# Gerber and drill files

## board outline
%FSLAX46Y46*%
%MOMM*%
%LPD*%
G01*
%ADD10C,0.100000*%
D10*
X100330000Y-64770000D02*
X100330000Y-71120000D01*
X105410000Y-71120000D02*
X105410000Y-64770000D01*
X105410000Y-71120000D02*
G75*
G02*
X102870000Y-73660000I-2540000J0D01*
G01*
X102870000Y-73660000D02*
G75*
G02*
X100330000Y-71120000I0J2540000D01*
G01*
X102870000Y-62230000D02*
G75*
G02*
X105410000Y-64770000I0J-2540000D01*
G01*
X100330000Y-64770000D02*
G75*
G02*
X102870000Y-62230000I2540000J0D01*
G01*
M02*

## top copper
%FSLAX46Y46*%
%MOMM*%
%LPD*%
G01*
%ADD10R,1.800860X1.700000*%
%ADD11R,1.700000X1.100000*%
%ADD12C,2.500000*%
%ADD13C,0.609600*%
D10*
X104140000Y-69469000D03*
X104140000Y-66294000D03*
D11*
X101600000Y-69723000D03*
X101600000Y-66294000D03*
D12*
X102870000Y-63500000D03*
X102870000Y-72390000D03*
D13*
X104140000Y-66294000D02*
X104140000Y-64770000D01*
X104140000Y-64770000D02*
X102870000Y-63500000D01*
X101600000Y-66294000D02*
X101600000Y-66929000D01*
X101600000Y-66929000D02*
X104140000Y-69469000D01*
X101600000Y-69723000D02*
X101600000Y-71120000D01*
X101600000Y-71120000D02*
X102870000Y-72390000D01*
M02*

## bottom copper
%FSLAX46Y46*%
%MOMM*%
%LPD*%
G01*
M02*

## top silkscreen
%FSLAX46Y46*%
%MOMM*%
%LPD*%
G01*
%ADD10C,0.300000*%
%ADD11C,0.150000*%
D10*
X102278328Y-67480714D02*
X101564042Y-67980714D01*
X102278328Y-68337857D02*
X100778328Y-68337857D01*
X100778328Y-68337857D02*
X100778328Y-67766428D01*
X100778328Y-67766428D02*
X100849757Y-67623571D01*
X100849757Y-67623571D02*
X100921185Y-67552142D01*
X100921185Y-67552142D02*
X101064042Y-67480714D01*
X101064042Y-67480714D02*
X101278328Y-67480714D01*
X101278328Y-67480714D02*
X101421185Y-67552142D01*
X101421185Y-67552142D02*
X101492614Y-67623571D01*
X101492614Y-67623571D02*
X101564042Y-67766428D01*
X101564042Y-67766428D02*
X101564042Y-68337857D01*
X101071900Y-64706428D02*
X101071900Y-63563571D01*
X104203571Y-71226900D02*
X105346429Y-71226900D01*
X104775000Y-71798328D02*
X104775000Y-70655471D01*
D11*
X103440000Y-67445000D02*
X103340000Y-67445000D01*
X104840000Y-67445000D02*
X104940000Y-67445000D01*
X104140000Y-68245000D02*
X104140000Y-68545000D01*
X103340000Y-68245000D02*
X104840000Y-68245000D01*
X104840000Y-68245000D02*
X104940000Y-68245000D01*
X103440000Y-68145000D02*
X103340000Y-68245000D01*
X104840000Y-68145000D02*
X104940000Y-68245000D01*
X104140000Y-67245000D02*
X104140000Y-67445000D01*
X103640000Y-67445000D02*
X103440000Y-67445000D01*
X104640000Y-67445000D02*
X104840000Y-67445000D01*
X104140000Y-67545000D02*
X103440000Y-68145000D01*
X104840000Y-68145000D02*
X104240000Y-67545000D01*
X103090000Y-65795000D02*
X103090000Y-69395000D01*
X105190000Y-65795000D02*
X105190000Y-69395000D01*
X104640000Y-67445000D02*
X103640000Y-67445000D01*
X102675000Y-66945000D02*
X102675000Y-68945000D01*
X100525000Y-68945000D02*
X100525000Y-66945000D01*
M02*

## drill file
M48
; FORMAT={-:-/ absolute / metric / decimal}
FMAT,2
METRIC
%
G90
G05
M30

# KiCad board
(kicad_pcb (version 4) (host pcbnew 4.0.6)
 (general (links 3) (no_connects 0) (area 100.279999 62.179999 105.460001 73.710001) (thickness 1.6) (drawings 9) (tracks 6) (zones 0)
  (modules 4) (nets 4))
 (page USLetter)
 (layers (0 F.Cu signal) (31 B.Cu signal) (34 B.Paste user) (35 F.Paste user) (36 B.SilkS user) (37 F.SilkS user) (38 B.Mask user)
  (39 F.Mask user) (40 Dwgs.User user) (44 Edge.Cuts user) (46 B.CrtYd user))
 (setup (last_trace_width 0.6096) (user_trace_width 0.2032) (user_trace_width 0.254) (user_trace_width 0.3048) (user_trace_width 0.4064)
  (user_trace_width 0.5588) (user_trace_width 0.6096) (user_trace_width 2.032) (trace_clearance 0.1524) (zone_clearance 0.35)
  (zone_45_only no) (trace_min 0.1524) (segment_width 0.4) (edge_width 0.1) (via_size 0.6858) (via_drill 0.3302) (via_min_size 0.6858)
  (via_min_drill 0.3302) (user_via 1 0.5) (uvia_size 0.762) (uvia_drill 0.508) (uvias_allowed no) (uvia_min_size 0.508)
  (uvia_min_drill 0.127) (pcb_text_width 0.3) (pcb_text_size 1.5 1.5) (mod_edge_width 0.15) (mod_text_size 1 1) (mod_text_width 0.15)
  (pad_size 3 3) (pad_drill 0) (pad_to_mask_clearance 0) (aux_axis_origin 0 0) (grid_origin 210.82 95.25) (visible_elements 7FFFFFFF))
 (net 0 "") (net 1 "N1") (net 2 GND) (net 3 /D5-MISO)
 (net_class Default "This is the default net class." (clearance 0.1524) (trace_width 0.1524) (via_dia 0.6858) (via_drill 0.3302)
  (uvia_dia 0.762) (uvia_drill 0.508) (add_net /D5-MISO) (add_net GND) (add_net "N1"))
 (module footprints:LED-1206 (layer F.Cu) (at 104.14 67.945 270)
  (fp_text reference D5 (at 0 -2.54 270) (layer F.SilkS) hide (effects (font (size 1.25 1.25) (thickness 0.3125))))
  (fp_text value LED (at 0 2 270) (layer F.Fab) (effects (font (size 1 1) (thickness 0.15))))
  (fp_line (start -0.5 0.7) (end -0.5 0.8) (layer F.SilkS) (width 0.15))
  (fp_line (start -0.5 -0.7) (end -0.5 -0.8) (layer F.SilkS) (width 0.15))
  (fp_line (start 0.3 0) (end 0.6 0) (layer F.SilkS) (width 0.15))
  (fp_line (start 0.3 0.8) (end 0.3 -0.7) (layer F.SilkS) (width 0.15))
  (fp_line (start 0.3 -0.7) (end 0.3 -0.8) (layer F.SilkS) (width 0.15))
  (fp_line (start 0.2 0.7) (end 0.3 0.8) (layer F.SilkS) (width 0.15))
  (fp_line (start 0.2 -0.7) (end 0.3 -0.8) (layer F.SilkS) (width 0.15))
  (fp_line (start -0.7 0) (end -0.5 0) (layer F.SilkS) (width 0.15))
  (fp_line (start -0.5 0.5) (end -0.5 0.7) (layer F.SilkS) (width 0.15))
  (fp_line (start -0.5 -0.5) (end -0.5 -0.7) (layer F.SilkS) (width 0.15))
  (fp_line (start -0.4 0) (end 0.2 0.7) (layer F.SilkS) (width 0.15))
  (fp_line (start 0.2 -0.7) (end -0.4 -0.1) (layer F.SilkS) (width 0.15))
  (fp_line (start -2.15 1.05) (end 1.45 1.05) (layer F.SilkS) (width 0.15))
  (fp_line (start -2.15 -1.05) (end 1.45 -1.05) (layer F.SilkS) (width 0.15))
  (fp_line (start -0.5 -0.5) (end -0.5 0.5) (layer F.SilkS) (width 0.15))
  (pad 2 smd rect (at 1.524 0 90) (size 1.7 1.80086) (layers F.Cu F.Paste F.Mask) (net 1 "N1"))
  (pad 1 smd rect (at -1.651 0 90) (size 1.7 1.80086) (layers F.Cu F.Paste F.Mask) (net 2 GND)))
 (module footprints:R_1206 (layer F.Cu) (at 101.6 67.945 90)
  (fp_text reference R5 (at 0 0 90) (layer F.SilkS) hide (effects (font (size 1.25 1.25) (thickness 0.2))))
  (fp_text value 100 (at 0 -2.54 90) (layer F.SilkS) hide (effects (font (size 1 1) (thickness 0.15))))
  (fp_line (start 1 1.075) (end -1 1.075) (layer F.SilkS) (width 0.15))
  (fp_line (start -1 -1.075) (end 1 -1.075) (layer F.SilkS) (width 0.15))
  (pad 1 smd rect (at -1.778 0 90) (size 1.1 1.7) (layers F.Cu F.Paste F.Mask) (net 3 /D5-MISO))
  (pad 2 smd rect (at 1.651 0 90) (size 1.1 1.7) (layers F.Cu F.Paste F.Mask) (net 1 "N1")))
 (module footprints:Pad (layer F.Cu) (at 102.87 63.5)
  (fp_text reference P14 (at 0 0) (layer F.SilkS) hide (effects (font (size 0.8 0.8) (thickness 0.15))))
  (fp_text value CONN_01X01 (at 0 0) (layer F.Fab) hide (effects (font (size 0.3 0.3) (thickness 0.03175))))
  (pad 1 smd circle (at 0 0) (size 2.5 2.5) (layers F.Cu F.Paste F.Mask) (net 2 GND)))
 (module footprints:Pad (layer F.Cu) (at 102.87 72.39)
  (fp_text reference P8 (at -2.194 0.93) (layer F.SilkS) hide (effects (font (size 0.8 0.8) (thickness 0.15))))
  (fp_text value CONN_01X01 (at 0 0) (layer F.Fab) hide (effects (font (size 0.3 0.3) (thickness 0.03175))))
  (pad 1 smd circle (at 0 0) (size 2.5 2.5) (layers F.Cu F.Paste F.Mask) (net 3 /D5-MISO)))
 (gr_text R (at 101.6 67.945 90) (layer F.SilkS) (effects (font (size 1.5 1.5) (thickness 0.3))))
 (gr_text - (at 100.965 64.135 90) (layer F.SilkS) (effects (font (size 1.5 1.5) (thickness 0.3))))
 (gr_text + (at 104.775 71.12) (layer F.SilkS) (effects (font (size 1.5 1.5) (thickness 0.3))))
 (gr_line (start 100.33 64.77) (end 100.33 71.12) (angle 90) (layer Edge.Cuts) (width 0.1))
 (gr_line (start 105.41 71.12) (end 105.41 64.77) (angle 90) (layer Edge.Cuts) (width 0.1))
 (gr_arc (start 102.87 71.12) (end 105.41 71.12) (angle 90) (layer Edge.Cuts) (width 0.1))
 (gr_arc (start 102.87 71.12) (end 102.87 73.66) (angle 90) (layer Edge.Cuts) (width 0.1))
 (gr_arc (start 102.87 64.77) (end 102.87 62.23) (angle 90) (layer Edge.Cuts) (width 0.1))
 (gr_arc (start 102.87 64.77) (end 100.33 64.77) (angle 90) (layer Edge.Cuts) (width 0.1))
 (segment (start 104.14 66.294) (end 104.14 64.77) (width 0.6096) (layer F.Cu) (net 2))
 (segment (start 104.14 64.77) (end 102.87 63.5) (width 0.6096) (layer F.Cu) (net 2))
 (segment (start 101.6 66.294) (end 101.6 66.929) (width 0.6096) (layer F.Cu) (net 1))
 (segment (start 101.6 66.929) (end 104.14 69.469) (width 0.6096) (layer F.Cu) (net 1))
 (segment (start 101.6 69.723) (end 101.6 71.12) (width 0.6096) (layer F.Cu) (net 3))
 (segment (start 101.6 71.12) (end 102.87 72.39) (width 0.6096) (layer F.Cu) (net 3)))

